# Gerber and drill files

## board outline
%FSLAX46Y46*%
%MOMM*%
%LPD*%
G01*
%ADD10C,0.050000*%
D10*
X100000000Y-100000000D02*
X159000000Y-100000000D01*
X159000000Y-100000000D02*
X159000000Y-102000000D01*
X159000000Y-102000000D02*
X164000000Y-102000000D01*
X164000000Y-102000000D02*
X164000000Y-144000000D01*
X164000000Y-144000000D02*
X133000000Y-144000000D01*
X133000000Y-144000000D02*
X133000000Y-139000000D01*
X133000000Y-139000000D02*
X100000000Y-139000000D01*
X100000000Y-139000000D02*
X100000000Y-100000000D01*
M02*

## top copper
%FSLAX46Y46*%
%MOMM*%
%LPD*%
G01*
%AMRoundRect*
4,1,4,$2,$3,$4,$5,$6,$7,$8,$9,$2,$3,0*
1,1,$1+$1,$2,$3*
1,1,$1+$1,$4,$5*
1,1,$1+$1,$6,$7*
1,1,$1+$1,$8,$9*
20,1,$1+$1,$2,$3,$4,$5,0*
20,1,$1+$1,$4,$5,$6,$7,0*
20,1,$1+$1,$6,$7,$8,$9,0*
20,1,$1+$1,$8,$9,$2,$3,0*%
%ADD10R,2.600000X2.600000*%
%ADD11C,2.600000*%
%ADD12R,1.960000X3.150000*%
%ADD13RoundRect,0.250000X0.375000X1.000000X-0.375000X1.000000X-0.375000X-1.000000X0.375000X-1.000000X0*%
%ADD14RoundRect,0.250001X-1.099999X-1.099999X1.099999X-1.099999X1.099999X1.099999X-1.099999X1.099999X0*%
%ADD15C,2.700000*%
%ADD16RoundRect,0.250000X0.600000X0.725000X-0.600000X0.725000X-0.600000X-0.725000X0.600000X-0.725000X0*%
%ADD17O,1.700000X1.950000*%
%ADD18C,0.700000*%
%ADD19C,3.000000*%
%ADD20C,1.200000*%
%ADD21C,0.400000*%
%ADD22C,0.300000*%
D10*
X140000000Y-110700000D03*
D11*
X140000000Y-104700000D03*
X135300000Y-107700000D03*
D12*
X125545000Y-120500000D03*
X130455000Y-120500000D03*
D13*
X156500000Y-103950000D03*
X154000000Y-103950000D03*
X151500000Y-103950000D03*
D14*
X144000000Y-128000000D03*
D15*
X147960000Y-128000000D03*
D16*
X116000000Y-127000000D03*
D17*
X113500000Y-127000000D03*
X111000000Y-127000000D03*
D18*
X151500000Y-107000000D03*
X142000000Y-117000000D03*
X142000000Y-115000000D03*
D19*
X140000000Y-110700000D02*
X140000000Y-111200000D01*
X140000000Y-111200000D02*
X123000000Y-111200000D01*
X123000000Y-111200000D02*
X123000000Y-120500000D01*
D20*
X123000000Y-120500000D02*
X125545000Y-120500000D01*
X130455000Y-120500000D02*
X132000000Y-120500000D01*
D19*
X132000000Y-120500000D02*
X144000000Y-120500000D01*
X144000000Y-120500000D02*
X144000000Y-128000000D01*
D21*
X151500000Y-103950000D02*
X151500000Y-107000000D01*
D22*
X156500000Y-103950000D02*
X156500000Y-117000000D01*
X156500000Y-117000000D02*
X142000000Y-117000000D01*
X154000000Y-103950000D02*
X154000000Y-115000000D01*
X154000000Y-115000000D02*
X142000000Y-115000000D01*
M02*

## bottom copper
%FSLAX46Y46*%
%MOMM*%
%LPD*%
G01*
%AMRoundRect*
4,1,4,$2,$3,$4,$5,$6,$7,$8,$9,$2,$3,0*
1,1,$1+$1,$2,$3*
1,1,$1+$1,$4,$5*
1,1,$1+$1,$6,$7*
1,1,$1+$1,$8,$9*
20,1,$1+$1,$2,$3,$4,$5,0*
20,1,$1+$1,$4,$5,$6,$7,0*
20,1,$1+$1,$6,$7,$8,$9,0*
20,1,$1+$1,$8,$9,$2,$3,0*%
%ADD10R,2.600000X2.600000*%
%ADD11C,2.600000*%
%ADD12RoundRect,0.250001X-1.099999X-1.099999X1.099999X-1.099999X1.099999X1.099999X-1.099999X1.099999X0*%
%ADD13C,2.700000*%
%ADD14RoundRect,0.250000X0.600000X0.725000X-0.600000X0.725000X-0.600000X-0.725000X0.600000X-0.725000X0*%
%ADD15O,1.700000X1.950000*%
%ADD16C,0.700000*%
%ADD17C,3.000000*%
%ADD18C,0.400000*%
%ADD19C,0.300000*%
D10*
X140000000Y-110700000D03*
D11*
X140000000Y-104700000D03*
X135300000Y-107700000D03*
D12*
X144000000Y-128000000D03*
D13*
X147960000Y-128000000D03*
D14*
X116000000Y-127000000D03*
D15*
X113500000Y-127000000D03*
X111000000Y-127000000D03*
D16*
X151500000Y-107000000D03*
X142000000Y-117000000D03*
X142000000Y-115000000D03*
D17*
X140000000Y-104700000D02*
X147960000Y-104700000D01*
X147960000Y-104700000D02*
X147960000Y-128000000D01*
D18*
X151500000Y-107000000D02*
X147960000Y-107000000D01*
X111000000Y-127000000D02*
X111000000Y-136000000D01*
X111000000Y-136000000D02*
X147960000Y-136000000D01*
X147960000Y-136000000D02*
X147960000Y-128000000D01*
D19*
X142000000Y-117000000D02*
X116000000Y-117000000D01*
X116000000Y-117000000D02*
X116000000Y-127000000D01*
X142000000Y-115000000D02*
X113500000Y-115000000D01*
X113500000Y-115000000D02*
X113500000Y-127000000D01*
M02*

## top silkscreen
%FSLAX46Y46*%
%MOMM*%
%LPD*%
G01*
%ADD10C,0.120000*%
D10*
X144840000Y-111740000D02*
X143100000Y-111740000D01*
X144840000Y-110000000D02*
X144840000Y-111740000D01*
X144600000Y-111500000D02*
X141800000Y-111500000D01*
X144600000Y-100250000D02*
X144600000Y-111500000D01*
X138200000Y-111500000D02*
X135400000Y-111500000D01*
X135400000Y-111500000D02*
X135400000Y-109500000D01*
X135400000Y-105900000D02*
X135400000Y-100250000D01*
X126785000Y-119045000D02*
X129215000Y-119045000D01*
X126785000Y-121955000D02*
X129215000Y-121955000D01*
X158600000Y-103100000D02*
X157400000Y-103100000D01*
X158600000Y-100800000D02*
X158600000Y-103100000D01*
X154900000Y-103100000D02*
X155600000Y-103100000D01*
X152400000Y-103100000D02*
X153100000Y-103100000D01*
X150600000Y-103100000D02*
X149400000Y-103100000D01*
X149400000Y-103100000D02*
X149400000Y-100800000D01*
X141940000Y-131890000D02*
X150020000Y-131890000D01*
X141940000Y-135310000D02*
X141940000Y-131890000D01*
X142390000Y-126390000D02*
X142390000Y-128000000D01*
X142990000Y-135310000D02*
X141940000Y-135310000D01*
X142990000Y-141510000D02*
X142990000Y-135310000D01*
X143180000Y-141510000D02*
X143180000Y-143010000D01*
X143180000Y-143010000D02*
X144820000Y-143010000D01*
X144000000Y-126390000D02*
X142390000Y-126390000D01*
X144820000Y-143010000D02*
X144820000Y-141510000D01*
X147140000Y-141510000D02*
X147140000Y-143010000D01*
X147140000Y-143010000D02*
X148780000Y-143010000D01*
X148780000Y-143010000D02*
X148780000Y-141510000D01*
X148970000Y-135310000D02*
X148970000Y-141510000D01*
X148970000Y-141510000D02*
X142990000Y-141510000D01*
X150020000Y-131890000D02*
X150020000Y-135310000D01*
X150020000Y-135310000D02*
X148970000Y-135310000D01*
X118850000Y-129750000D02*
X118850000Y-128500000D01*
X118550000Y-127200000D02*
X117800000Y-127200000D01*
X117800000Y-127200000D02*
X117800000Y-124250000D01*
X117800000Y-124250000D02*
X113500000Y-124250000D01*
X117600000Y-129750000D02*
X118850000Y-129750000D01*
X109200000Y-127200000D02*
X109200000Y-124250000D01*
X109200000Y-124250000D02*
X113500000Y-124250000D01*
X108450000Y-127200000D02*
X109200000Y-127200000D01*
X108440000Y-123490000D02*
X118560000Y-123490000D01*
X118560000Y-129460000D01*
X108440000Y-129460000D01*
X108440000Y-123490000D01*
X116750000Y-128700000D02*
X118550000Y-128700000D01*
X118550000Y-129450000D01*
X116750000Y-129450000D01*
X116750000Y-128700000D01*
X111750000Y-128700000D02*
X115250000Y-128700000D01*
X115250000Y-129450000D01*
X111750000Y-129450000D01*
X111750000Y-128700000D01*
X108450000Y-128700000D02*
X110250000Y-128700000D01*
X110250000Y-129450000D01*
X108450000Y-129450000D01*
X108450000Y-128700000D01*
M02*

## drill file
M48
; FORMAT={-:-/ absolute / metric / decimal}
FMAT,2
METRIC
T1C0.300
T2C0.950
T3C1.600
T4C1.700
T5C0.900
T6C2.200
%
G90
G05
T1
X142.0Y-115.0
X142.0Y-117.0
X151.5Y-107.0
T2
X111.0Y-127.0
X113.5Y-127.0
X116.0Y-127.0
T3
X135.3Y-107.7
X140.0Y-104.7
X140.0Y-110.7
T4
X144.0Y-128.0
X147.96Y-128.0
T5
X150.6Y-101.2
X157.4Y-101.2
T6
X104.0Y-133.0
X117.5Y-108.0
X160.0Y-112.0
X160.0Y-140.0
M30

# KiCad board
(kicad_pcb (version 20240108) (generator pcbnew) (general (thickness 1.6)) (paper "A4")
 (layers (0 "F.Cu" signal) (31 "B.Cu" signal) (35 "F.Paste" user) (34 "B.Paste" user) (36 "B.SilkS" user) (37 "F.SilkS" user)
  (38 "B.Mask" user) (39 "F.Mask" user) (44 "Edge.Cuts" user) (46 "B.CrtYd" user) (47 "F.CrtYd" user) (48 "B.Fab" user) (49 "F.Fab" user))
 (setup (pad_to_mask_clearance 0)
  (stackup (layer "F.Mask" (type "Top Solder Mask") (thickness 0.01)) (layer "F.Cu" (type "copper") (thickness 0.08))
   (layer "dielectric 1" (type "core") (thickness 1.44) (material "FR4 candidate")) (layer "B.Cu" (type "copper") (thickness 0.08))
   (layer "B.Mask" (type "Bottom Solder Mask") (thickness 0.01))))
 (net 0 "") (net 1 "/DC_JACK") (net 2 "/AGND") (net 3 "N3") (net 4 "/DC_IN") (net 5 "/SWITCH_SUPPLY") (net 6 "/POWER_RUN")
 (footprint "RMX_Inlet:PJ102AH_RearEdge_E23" (layer "F.Cu")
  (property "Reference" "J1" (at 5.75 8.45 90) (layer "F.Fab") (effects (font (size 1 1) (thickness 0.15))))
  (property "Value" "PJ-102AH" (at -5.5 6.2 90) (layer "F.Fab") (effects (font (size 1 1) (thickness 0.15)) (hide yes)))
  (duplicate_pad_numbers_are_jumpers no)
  (fp_line (start -4.84 -1.04) (end -3.1 -1.04) (stroke (width 0.12) (type solid)) (layer "F.SilkS"))
  (fp_line (start -4.84 0.7) (end -4.84 -1.04) (stroke (width 0.12) (type solid)) (layer "F.SilkS"))
  (fp_line (start -4.6 -0.8) (end -1.8 -0.8) (stroke (width 0.12) (type solid)) (layer "F.SilkS"))
  (fp_line (start -4.6 10.45) (end -4.6 -0.8) (stroke (width 0.12) (type solid)) (layer "F.SilkS"))
  (fp_line (start 1.8 -0.8) (end 4.6 -0.8) (stroke (width 0.12) (type solid)) (layer "F.SilkS"))
  (fp_line (start 4.6 -0.8) (end 4.6 1.2) (stroke (width 0.12) (type solid)) (layer "F.SilkS"))
  (fp_line (start 4.6 4.8) (end 4.6 10.45) (stroke (width 0.12) (type solid)) (layer "F.SilkS"))
  (pad "1" thru_hole rect (at 0 0) (size 2.6 2.6) (drill 1.6) (layers "*.Cu" "*.Mask") (remove_unused_layers no) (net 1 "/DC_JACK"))
  (pad "2" thru_hole circle (at 0 6) (size 2.6 2.6) (drill 1.6) (layers "*.Cu" "*.Mask") (remove_unused_layers no) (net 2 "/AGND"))
  (pad "3" thru_hole circle (at 4.7 3) (size 2.6 2.6) (drill 1.6) (layers "*.Cu" "*.Mask") (remove_unused_layers no) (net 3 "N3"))
  (at 140 110.7 180))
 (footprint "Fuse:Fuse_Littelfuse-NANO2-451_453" (layer "F.Cu")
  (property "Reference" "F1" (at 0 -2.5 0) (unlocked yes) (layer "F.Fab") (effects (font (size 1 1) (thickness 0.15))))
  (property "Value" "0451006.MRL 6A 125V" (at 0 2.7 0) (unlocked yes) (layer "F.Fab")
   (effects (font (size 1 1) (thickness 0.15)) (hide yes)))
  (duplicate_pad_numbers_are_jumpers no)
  (fp_line (start -1.215 -1.455) (end 1.215 -1.455) (stroke (width 0.12) (type solid)) (layer "F.SilkS"))
  (fp_line (start -1.215 1.455) (end 1.215 1.455) (stroke (width 0.12) (type solid)) (layer "F.SilkS"))
  (pad "1" smd rect (at -2.455 0) (size 1.96 3.15) (layers "F.Cu" "F.Mask" "F.Paste") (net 1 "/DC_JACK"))
  (pad "2" smd rect (at 2.455 0) (size 1.96 3.15) (layers "F.Cu" "F.Mask" "F.Paste") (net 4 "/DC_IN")) (at 128 120.5 0))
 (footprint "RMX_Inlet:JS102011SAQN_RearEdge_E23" (layer "F.Cu")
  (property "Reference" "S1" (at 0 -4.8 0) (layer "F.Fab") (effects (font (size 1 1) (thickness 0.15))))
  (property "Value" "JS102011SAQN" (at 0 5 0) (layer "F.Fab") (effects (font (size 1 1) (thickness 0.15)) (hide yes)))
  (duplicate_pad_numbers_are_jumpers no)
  (fp_line (start -4.6 -1.9) (end -3.4 -1.9) (stroke (width 0.12) (type solid)) (layer "F.SilkS"))
  (fp_line (start -4.6 0.4) (end -4.6 -1.9) (stroke (width 0.12) (type solid)) (layer "F.SilkS"))
  (fp_line (start -0.9 -1.9) (end -1.6 -1.9) (stroke (width 0.12) (type solid)) (layer "F.SilkS"))
  (fp_line (start 1.6 -1.9) (end 0.9 -1.9) (stroke (width 0.12) (type solid)) (layer "F.SilkS"))
  (fp_line (start 3.4 -1.9) (end 4.6 -1.9) (stroke (width 0.12) (type solid)) (layer "F.SilkS"))
  (fp_line (start 4.6 -1.9) (end 4.6 0.4) (stroke (width 0.12) (type solid)) (layer "F.SilkS"))
  (pad "" np_thru_hole circle (at -3.4 0) (size 0.9 0.9) (drill 0.9) (layers "*.Cu" "*.Mask"))
  (pad "" np_thru_hole circle (at 3.4 0) (size 0.9 0.9) (drill 0.9) (layers "*.Cu" "*.Mask"))
  (pad "1" smd roundrect (at -2.5 -2.75) (size 1.25 2.5) (layers "F.Cu" "F.Mask" "F.Paste") (roundrect_rratio 0.2) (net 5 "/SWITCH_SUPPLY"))
  (pad "2" smd roundrect (at 0 -2.75) (size 1.25 2.5) (layers "F.Cu" "F.Mask" "F.Paste") (roundrect_rratio 0.2) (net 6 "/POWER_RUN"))
  (pad "3" smd roundrect (at 2.5 -2.75) (size 1.25 2.5) (layers "F.Cu" "F.Mask" "F.Paste") (roundrect_rratio 0.2) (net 2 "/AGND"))
  (at 154 101.2 180))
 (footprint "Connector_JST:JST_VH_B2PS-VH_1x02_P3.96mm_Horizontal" (layer "F.Cu")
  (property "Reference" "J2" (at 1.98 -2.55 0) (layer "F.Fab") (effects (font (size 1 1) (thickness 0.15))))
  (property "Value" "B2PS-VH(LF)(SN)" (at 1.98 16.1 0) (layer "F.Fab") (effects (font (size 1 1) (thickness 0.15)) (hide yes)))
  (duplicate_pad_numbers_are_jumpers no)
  (fp_line (start -2.06 3.89) (end 6.02 3.89) (stroke (width 0.12) (type solid)) (layer "F.SilkS"))
  (fp_line (start -2.06 7.31) (end -2.06 3.89) (stroke (width 0.12) (type solid)) (layer "F.SilkS"))
  (fp_line (start -1.61 -1.61) (end -1.61 0) (stroke (width 0.12) (type solid)) (layer "F.SilkS"))
  (fp_line (start -1.01 7.31) (end -2.06 7.31) (stroke (width 0.12) (type solid)) (layer "F.SilkS"))
  (fp_line (start -1.01 13.51) (end -1.01 7.31) (stroke (width 0.12) (type solid)) (layer "F.SilkS"))
  (fp_line (start -0.82 13.51) (end -0.82 15.01) (stroke (width 0.12) (type solid)) (layer "F.SilkS"))
  (fp_line (start -0.82 15.01) (end 0.82 15.01) (stroke (width 0.12) (type solid)) (layer "F.SilkS"))
  (fp_line (start 0 -1.61) (end -1.61 -1.61) (stroke (width 0.12) (type solid)) (layer "F.SilkS"))
  (fp_line (start 0.82 15.01) (end 0.82 13.51) (stroke (width 0.12) (type solid)) (layer "F.SilkS"))
  (fp_line (start 3.14 13.51) (end 3.14 15.01) (stroke (width 0.12) (type solid)) (layer "F.SilkS"))
  (fp_line (start 3.14 15.01) (end 4.78 15.01) (stroke (width 0.12) (type solid)) (layer "F.SilkS"))
  (fp_line (start 4.78 15.01) (end 4.78 13.51) (stroke (width 0.12) (type solid)) (layer "F.SilkS"))
  (fp_line (start 4.97 7.31) (end 4.97 13.51) (stroke (width 0.12) (type solid)) (layer "F.SilkS"))
  (fp_line (start 4.97 13.51) (end -1.01 13.51) (stroke (width 0.12) (type solid)) (layer "F.SilkS"))
  (fp_line (start 6.02 3.89) (end 6.02 7.31) (stroke (width 0.12) (type solid)) (layer "F.SilkS"))
  (fp_line (start 6.02 7.31) (end 4.97 7.31) (stroke (width 0.12) (type solid)) (layer "F.SilkS"))
  (pad "1" thru_hole roundrect (at 0 0) (size 2.7 2.7) (drill 1.7) (layers "*.Cu" "*.Mask") (remove_unused_layers no)
   (roundrect_rratio 0.092593) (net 4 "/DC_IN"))
  (pad "2" thru_hole circle (at 3.96 0) (size 2.7 2.7) (drill 1.7) (layers "*.Cu" "*.Mask") (remove_unused_layers no) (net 2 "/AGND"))
  (at 144 128 0))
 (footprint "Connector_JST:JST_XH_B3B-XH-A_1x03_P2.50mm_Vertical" (layer "F.Cu")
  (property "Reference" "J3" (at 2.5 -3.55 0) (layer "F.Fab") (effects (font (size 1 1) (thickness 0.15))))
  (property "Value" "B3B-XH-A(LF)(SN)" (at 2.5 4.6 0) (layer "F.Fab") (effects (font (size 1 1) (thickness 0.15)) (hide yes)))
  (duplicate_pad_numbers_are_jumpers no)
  (fp_line (start -2.85 -2.75) (end -2.85 -1.5) (stroke (width 0.12) (type solid)) (layer "F.SilkS"))
  (fp_line (start -2.55 -0.2) (end -1.8 -0.2) (stroke (width 0.12) (type solid)) (layer "F.SilkS"))
  (fp_line (start -1.8 -0.2) (end -1.8 2.75) (stroke (width 0.12) (type solid)) (layer "F.SilkS"))
  (fp_line (start -1.8 2.75) (end 2.5 2.75) (stroke (width 0.12) (type solid)) (layer "F.SilkS"))
  (fp_line (start -1.6 -2.75) (end -2.85 -2.75) (stroke (width 0.12) (type solid)) (layer "F.SilkS"))
  (fp_line (start 6.8 -0.2) (end 6.8 2.75) (stroke (width 0.12) (type solid)) (layer "F.SilkS"))
  (fp_line (start 6.8 2.75) (end 2.5 2.75) (stroke (width 0.12) (type solid)) (layer "F.SilkS"))
  (fp_line (start 7.55 -0.2) (end 6.8 -0.2) (stroke (width 0.12) (type solid)) (layer "F.SilkS"))
  (fp_rect (start -2.56 -2.46) (end 7.56 3.51) (stroke (width 0.12) (type solid)) (fill no) (layer "F.SilkS"))
  (fp_rect (start -2.55 -2.45) (end -0.75 -1.7) (stroke (width 0.12) (type solid)) (fill no) (layer "F.SilkS"))
  (fp_rect (start 0.75 -2.45) (end 4.25 -1.7) (stroke (width 0.12) (type solid)) (fill no) (layer "F.SilkS"))
  (fp_rect (start 5.75 -2.45) (end 7.55 -1.7) (stroke (width 0.12) (type solid)) (fill no) (layer "F.SilkS"))
  (pad "1" thru_hole roundrect (at 0 0) (size 1.7 1.95) (drill 0.95) (layers "*.Cu" "*.Mask") (remove_unused_layers no)
   (roundrect_rratio 0.147059) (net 5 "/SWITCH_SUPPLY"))
  (pad "2" thru_hole oval (at 2.5 0) (size 1.7 1.95) (drill 0.95) (layers "*.Cu" "*.Mask") (remove_unused_layers no) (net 6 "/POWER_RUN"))
  (pad "3" thru_hole oval (at 5 0) (size 1.7 1.95) (drill 0.95) (layers "*.Cu" "*.Mask") (remove_unused_layers no) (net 2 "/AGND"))
  (at 116 127 180))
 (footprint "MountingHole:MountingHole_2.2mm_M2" (layer "F.Cu")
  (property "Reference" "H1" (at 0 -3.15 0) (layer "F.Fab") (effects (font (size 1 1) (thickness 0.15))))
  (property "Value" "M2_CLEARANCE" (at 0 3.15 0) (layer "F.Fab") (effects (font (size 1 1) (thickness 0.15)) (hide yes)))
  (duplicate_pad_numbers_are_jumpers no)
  (pad "" np_thru_hole circle (at 0 0) (size 2.2 2.2) (drill 2.2) (layers "*.Cu" "*.Mask")) (at 117.5 108 0))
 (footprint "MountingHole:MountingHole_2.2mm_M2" (layer "F.Cu")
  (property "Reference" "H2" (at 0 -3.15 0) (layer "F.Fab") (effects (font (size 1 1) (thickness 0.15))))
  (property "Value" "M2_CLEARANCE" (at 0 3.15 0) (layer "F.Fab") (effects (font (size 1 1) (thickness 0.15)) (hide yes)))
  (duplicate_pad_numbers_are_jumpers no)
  (pad "" np_thru_hole circle (at 0 0) (size 2.2 2.2) (drill 2.2) (layers "*.Cu" "*.Mask")) (at 160 112 0))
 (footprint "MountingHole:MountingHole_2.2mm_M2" (layer "F.Cu")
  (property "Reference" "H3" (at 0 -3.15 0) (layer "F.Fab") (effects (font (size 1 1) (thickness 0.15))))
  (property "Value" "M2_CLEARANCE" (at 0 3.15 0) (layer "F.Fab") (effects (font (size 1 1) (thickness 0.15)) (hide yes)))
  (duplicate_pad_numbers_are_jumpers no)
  (pad "" np_thru_hole circle (at 0 0) (size 2.2 2.2) (drill 2.2) (layers "*.Cu" "*.Mask")) (at 104 133 0))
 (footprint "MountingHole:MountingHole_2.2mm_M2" (layer "F.Cu")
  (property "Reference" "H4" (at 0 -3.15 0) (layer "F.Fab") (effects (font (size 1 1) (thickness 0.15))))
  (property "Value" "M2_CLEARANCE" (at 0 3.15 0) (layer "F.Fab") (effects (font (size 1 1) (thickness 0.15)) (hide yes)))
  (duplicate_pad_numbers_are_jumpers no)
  (pad "" np_thru_hole circle (at 0 0) (size 2.2 2.2) (drill 2.2) (layers "*.Cu" "*.Mask")) (at 160 140 0))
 (gr_line (start 100 100) (end 159 100) (stroke (width .05) (type default)) (layer "Edge.Cuts"))
 (gr_line (start 159 100) (end 159 102) (stroke (width .05) (type default)) (layer "Edge.Cuts"))
 (gr_line (start 159 102) (end 164 102) (stroke (width .05) (type default)) (layer "Edge.Cuts"))
 (gr_line (start 164 102) (end 164 144) (stroke (width .05) (type default)) (layer "Edge.Cuts"))
 (gr_line (start 164 144) (end 133 144) (stroke (width .05) (type default)) (layer "Edge.Cuts"))
 (gr_line (start 133 144) (end 133 139) (stroke (width .05) (type default)) (layer "Edge.Cuts"))
 (gr_line (start 133 139) (end 100 139) (stroke (width .05) (type default)) (layer "Edge.Cuts"))
 (gr_line (start 100 139) (end 100 100) (stroke (width .05) (type default)) (layer "Edge.Cuts"))
 (segment (start 140.0 110.7) (end 140 111.2) (width 3) (layer "F.Cu") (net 1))
 (segment (start 140 111.2) (end 123 111.2) (width 3) (layer "F.Cu") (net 1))
 (segment (start 123 111.2) (end 123 120.5) (width 3) (layer "F.Cu") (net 1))
 (segment (start 123 120.5) (end 125.545 120.5) (width 1.2) (layer "F.Cu") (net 1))
 (segment (start 130.455 120.5) (end 132 120.5) (width 1.2) (layer "F.Cu") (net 4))
 (segment (start 132 120.5) (end 144 120.5) (width 3) (layer "F.Cu") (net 4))
 (segment (start 144 120.5) (end 144.0 128.0) (width 3) (layer "F.Cu") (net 4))
 (segment (start 140.0 104.7) (end 147.96 104.7) (width 3) (layer "B.Cu") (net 2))
 (segment (start 147.96 104.7) (end 147.96 128.0) (width 3) (layer "B.Cu") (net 2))
 (segment (start 151.5 103.95) (end 151.5 107) (width 0.4) (layer "F.Cu") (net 2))
 (via (at 151.5 107) (size .7) (drill .3) (layers "F.Cu" "B.Cu") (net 2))
 (segment (start 151.5 107) (end 147.96 107) (width 0.4) (layer "B.Cu") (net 2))
 (segment (start 111.0 127.0) (end 111 136) (width 0.4) (layer "B.Cu") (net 2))
 (segment (start 111 136) (end 147.96 136) (width 0.4) (layer "B.Cu") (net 2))
 (segment (start 147.96 136) (end 147.96 128.0) (width 0.4) (layer "B.Cu") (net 2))
 (segment (start 156.5 103.95) (end 156.5 117) (width 0.3) (layer "F.Cu") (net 5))
 (segment (start 156.5 117) (end 142 117) (width 0.3) (layer "F.Cu") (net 5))
 (via (at 142 117) (size .7) (drill .3) (layers "F.Cu" "B.Cu") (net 5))
 (segment (start 142 117) (end 116.0 117) (width 0.3) (layer "B.Cu") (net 5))
 (segment (start 116.0 117) (end 116.0 127.0) (width 0.3) (layer "B.Cu") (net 5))
 (segment (start 154.0 103.95) (end 154.0 115) (width 0.3) (layer "F.Cu") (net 6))
 (segment (start 154.0 115) (end 142 115) (width 0.3) (layer "F.Cu") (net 6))
 (via (at 142 115) (size .7) (drill .3) (layers "F.Cu" "B.Cu") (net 6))
 (segment (start 142 115) (end 113.5 115) (width 0.3) (layer "B.Cu") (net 6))
 (segment (start 113.5 115) (end 113.5 127.0) (width 0.3) (layer "B.Cu") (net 6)))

